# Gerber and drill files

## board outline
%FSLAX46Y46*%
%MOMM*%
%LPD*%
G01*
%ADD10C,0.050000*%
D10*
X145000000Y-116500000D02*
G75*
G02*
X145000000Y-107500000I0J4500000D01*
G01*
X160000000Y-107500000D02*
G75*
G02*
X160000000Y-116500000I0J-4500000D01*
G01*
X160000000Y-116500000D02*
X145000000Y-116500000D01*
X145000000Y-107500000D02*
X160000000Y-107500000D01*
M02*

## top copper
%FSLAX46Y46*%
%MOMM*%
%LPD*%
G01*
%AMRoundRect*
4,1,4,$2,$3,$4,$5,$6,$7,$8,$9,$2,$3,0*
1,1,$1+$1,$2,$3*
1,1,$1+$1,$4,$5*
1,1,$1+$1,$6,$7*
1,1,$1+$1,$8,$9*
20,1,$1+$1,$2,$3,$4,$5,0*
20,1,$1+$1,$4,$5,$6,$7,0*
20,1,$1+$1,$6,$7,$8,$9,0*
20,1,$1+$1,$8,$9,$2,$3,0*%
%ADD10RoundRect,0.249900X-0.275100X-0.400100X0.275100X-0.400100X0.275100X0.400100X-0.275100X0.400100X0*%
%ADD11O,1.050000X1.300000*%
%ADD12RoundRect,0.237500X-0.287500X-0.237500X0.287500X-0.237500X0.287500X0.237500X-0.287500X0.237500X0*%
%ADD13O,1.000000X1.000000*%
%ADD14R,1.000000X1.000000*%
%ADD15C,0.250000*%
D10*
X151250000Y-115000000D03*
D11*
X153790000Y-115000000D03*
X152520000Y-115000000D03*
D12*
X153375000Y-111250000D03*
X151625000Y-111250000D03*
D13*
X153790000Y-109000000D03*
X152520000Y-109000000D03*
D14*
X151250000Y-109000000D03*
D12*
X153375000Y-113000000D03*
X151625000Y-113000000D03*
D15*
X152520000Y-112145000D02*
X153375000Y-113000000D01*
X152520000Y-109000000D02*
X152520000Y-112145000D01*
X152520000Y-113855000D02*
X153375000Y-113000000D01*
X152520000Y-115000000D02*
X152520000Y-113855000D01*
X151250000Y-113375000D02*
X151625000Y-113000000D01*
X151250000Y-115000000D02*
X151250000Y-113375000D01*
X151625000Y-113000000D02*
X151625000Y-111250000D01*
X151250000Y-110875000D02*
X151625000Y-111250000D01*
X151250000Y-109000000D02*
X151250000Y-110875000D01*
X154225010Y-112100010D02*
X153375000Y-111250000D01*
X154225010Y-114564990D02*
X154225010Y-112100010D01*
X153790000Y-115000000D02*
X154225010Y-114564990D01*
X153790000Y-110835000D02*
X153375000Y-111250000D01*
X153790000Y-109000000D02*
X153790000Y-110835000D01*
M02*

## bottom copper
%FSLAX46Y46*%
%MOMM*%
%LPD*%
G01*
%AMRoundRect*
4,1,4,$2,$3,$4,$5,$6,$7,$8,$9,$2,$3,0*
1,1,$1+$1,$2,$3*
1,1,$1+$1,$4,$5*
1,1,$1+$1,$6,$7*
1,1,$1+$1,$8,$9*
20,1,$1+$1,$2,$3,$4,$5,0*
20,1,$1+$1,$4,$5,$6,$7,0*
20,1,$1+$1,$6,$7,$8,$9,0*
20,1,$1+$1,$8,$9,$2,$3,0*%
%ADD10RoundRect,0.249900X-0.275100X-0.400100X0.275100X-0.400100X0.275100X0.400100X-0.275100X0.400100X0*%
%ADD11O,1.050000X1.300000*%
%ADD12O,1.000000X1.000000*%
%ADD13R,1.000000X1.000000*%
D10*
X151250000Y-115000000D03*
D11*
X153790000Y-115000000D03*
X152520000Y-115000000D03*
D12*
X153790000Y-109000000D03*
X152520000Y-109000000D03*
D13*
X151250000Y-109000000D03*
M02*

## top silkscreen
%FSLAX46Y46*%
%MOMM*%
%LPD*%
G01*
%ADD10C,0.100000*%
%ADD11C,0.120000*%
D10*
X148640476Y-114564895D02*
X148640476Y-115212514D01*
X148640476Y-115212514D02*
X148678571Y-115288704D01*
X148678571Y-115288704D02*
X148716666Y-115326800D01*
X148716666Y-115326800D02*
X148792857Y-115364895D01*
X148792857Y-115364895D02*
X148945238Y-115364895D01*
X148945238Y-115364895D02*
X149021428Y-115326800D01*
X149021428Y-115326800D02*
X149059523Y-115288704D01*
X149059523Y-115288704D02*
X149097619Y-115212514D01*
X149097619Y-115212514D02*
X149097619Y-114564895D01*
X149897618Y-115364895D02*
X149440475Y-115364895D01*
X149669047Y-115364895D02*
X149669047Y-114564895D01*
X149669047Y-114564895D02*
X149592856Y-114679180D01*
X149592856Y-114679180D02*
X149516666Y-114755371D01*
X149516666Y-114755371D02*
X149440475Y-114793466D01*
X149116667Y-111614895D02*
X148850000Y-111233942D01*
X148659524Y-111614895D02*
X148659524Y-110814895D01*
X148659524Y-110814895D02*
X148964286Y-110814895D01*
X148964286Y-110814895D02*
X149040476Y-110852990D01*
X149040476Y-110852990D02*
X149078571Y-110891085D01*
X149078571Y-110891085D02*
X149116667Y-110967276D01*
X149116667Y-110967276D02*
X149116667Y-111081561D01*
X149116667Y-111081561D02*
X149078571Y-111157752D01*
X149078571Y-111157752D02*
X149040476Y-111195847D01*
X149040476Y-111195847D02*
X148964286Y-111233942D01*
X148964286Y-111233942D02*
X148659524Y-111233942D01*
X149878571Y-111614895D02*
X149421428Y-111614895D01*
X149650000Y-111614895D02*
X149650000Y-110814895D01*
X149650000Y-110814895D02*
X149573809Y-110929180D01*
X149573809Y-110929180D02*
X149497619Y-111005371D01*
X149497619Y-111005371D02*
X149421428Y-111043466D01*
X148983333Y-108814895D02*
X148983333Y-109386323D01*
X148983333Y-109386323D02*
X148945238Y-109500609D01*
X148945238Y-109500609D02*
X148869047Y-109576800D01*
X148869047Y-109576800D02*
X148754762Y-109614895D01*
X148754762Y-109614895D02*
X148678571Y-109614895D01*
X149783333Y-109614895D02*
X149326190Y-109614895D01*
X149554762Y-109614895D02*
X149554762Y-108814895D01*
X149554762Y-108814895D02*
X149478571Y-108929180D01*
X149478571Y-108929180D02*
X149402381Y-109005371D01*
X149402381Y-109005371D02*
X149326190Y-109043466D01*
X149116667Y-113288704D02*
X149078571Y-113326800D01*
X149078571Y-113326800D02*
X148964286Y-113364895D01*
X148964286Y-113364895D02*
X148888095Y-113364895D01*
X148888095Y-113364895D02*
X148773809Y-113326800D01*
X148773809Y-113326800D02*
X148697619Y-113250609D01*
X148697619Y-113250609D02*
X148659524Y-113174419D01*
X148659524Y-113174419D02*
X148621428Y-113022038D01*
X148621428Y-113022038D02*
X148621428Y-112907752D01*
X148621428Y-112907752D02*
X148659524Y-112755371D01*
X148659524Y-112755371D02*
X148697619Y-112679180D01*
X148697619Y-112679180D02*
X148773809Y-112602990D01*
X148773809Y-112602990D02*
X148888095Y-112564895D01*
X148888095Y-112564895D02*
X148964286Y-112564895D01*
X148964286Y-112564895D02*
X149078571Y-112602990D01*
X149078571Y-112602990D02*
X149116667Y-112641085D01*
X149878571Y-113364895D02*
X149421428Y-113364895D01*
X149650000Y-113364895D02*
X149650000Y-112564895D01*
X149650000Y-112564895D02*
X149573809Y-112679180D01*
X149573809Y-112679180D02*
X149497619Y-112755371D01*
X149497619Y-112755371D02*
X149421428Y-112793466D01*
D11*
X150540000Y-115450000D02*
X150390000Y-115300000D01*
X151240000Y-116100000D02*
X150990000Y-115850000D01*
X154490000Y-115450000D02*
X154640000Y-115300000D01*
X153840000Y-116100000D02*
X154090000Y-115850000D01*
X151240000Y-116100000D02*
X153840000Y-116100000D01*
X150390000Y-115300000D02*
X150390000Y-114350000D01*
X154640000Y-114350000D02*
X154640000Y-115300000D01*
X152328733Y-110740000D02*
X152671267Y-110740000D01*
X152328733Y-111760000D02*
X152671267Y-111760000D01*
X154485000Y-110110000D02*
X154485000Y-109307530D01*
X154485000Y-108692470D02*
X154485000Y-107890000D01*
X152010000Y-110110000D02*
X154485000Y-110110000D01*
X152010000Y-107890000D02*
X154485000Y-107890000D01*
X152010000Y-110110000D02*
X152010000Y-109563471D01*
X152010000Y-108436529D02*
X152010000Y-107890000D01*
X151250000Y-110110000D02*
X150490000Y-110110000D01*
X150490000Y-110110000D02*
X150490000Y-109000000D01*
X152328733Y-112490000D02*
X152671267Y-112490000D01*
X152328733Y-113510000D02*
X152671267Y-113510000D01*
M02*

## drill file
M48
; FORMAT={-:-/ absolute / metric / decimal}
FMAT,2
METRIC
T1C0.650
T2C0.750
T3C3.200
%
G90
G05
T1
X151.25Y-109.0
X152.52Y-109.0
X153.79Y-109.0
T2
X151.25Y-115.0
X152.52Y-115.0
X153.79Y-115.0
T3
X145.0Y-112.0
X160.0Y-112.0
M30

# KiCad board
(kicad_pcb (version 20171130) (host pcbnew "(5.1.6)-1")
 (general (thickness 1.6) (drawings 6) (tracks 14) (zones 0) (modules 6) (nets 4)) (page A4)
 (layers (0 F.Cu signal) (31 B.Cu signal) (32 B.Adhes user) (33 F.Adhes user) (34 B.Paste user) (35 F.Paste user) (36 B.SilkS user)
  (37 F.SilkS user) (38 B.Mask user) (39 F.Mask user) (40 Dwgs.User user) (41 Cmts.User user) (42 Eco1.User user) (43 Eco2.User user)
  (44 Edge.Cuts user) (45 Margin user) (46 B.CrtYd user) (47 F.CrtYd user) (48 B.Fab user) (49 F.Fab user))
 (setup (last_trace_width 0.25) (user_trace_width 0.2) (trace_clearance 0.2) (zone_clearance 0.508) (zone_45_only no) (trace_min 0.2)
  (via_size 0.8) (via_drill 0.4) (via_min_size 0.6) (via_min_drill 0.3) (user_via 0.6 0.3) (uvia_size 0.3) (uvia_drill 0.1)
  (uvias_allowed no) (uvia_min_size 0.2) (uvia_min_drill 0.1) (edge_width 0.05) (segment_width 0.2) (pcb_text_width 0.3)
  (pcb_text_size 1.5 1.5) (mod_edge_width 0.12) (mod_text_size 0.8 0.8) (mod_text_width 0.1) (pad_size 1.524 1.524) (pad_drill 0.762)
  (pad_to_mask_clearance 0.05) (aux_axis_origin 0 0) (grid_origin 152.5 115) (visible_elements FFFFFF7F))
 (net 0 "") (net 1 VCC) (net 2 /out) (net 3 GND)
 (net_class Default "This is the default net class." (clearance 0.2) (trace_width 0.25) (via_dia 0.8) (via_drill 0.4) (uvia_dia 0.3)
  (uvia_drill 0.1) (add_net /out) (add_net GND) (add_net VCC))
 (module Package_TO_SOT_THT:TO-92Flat (layer F.Cu) (at 151.25 115)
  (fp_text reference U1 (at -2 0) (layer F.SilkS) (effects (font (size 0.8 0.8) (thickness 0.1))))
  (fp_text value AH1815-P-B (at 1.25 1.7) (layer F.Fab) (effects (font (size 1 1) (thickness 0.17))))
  (fp_line (start -0.71 0.45) (end -0.86 0.3) (layer F.SilkS) (width 0.12))
  (fp_line (start -0.01 1.1) (end -0.26 0.85) (layer F.SilkS) (width 0.12))
  (fp_line (start 3.24 0.45) (end 3.39 0.3) (layer F.SilkS) (width 0.12))
  (fp_line (start 2.59 1.1) (end 2.84 0.85) (layer F.SilkS) (width 0.12))
  (fp_line (start -0.01 1.1) (end 2.59 1.1) (layer F.SilkS) (width 0.12))
  (fp_line (start -0.86 0.3) (end -0.86 -0.65) (layer F.SilkS) (width 0.12))
  (fp_line (start 3.39 -0.65) (end 3.39 0.3) (layer F.SilkS) (width 0.12))
  (pad 1 thru_hole roundrect (at 0 0) (size 1.05 1.3) (drill 0.75) (layers *.Cu *.Mask) (roundrect_rratio 0.238) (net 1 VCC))
  (pad 3 thru_hole oval (at 2.54 0) (size 1.05 1.3) (drill 0.75) (layers *.Cu *.Mask) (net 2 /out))
  (pad 2 thru_hole oval (at 1.27 0) (size 1.05 1.3) (drill 0.75) (layers *.Cu *.Mask) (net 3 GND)))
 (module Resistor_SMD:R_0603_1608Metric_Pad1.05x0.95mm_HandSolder (layer F.Cu) (at 152.5 111.25)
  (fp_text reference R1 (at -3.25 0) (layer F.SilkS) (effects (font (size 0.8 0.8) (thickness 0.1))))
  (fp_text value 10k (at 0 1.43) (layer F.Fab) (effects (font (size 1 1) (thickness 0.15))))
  (fp_line (start -0.171267 -0.51) (end 0.171267 -0.51) (layer F.SilkS) (width 0.12))
  (fp_line (start -0.171267 0.51) (end 0.171267 0.51) (layer F.SilkS) (width 0.12))
  (pad 2 smd roundrect (at 0.875 0) (size 1.05 0.95) (layers F.Cu F.Paste F.Mask) (roundrect_rratio 0.25) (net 2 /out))
  (pad 1 smd roundrect (at -0.875 0) (size 1.05 0.95) (layers F.Cu F.Paste F.Mask) (roundrect_rratio 0.25) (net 1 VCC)))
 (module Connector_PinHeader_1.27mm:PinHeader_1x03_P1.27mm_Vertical (layer F.Cu) (at 151.25 109 90)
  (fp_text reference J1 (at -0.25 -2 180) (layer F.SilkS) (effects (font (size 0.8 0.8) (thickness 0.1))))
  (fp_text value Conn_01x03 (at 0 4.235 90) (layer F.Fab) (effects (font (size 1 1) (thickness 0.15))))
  (fp_line (start -1.11 3.235) (end -0.30753 3.235) (layer F.SilkS) (width 0.12))
  (fp_line (start 0.30753 3.235) (end 1.11 3.235) (layer F.SilkS) (width 0.12))
  (fp_line (start -1.11 0.76) (end -1.11 3.235) (layer F.SilkS) (width 0.12))
  (fp_line (start 1.11 0.76) (end 1.11 3.235) (layer F.SilkS) (width 0.12))
  (fp_line (start -1.11 0.76) (end -0.563471 0.76) (layer F.SilkS) (width 0.12))
  (fp_line (start 0.563471 0.76) (end 1.11 0.76) (layer F.SilkS) (width 0.12))
  (fp_line (start -1.11 0) (end -1.11 -0.76) (layer F.SilkS) (width 0.12))
  (fp_line (start -1.11 -0.76) (end 0 -0.76) (layer F.SilkS) (width 0.12))
  (pad 3 thru_hole oval (at 0 2.54 90) (size 1 1) (drill 0.65) (layers *.Cu *.Mask) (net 2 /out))
  (pad 2 thru_hole oval (at 0 1.27 90) (size 1 1) (drill 0.65) (layers *.Cu *.Mask) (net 3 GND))
  (pad 1 thru_hole rect (at 0 0 90) (size 1 1) (drill 0.65) (layers *.Cu *.Mask) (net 1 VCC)))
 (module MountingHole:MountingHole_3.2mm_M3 (layer F.Cu) (at 160 112)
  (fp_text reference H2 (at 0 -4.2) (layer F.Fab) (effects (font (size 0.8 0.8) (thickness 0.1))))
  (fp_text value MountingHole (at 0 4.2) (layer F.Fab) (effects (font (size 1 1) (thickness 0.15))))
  (pad 1 np_thru_hole circle (at 0 0) (size 3.2 3.2) (drill 3.2) (layers *.Cu *.Mask)))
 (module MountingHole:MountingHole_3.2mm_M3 (layer F.Cu) (at 145 112)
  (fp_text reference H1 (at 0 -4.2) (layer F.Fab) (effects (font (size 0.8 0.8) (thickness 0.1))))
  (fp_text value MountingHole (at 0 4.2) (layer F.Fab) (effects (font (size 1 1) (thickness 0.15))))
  (pad 1 np_thru_hole circle (at 0 0) (size 3.2 3.2) (drill 3.2) (layers *.Cu *.Mask)))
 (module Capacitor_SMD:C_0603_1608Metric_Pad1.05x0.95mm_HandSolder (layer F.Cu) (at 152.5 113)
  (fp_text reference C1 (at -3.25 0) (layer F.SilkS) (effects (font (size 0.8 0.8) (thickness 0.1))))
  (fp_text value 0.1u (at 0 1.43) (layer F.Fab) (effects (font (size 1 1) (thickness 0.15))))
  (fp_line (start -0.171267 -0.51) (end 0.171267 -0.51) (layer F.SilkS) (width 0.12))
  (fp_line (start -0.171267 0.51) (end 0.171267 0.51) (layer F.SilkS) (width 0.12))
  (pad 2 smd roundrect (at 0.875 0) (size 1.05 0.95) (layers F.Cu F.Paste F.Mask) (roundrect_rratio 0.25) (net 3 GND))
  (pad 1 smd roundrect (at -0.875 0) (size 1.05 0.95) (layers F.Cu F.Paste F.Mask) (roundrect_rratio 0.25) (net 1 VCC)))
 (gr_arc (start 145 112) (end 145 107.5) (angle -180) (layer Edge.Cuts) (width 0.05))
 (gr_arc (start 160 112) (end 160 116.5) (angle -180) (layer Edge.Cuts) (width 0.05))
 (gr_line (start 160 116.5) (end 145 116.5) (layer Edge.Cuts) (width 0.05))
 (gr_line (start 145 107.5) (end 160 107.5) (layer Edge.Cuts) (width 0.05))
 (segment (start 152.52 112.145) (end 153.375 113) (width 0.25) (layer F.Cu) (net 3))
 (segment (start 152.52 109) (end 152.52 112.145) (width 0.25) (layer F.Cu) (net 3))
 (segment (start 152.52 113.855) (end 153.375 113) (width 0.25) (layer F.Cu) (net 3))
 (segment (start 152.52 115) (end 152.52 113.855) (width 0.25) (layer F.Cu) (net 3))
 (segment (start 151.25 113.375) (end 151.625 113) (width 0.25) (layer F.Cu) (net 1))
 (segment (start 151.25 115) (end 151.25 113.375) (width 0.25) (layer F.Cu) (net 1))
 (segment (start 151.625 113) (end 151.625 111.25) (width 0.25) (layer F.Cu) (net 1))
 (segment (start 151.25 110.875) (end 151.625 111.25) (width 0.25) (layer F.Cu) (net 1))
 (segment (start 151.25 109) (end 151.25 110.875) (width 0.25) (layer F.Cu) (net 1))
 (segment (start 154.22501 112.10001) (end 153.375 111.25) (width 0.25) (layer F.Cu) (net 2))
 (segment (start 154.22501 114.56499) (end 154.22501 112.10001) (width 0.25) (layer F.Cu) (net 2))
 (segment (start 153.79 115) (end 154.22501 114.56499) (width 0.25) (layer F.Cu) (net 2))
 (segment (start 153.79 110.835) (end 153.375 111.25) (width 0.25) (layer F.Cu) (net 2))
 (segment (start 153.79 109) (end 153.79 110.835) (width 0.25) (layer F.Cu) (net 2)))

